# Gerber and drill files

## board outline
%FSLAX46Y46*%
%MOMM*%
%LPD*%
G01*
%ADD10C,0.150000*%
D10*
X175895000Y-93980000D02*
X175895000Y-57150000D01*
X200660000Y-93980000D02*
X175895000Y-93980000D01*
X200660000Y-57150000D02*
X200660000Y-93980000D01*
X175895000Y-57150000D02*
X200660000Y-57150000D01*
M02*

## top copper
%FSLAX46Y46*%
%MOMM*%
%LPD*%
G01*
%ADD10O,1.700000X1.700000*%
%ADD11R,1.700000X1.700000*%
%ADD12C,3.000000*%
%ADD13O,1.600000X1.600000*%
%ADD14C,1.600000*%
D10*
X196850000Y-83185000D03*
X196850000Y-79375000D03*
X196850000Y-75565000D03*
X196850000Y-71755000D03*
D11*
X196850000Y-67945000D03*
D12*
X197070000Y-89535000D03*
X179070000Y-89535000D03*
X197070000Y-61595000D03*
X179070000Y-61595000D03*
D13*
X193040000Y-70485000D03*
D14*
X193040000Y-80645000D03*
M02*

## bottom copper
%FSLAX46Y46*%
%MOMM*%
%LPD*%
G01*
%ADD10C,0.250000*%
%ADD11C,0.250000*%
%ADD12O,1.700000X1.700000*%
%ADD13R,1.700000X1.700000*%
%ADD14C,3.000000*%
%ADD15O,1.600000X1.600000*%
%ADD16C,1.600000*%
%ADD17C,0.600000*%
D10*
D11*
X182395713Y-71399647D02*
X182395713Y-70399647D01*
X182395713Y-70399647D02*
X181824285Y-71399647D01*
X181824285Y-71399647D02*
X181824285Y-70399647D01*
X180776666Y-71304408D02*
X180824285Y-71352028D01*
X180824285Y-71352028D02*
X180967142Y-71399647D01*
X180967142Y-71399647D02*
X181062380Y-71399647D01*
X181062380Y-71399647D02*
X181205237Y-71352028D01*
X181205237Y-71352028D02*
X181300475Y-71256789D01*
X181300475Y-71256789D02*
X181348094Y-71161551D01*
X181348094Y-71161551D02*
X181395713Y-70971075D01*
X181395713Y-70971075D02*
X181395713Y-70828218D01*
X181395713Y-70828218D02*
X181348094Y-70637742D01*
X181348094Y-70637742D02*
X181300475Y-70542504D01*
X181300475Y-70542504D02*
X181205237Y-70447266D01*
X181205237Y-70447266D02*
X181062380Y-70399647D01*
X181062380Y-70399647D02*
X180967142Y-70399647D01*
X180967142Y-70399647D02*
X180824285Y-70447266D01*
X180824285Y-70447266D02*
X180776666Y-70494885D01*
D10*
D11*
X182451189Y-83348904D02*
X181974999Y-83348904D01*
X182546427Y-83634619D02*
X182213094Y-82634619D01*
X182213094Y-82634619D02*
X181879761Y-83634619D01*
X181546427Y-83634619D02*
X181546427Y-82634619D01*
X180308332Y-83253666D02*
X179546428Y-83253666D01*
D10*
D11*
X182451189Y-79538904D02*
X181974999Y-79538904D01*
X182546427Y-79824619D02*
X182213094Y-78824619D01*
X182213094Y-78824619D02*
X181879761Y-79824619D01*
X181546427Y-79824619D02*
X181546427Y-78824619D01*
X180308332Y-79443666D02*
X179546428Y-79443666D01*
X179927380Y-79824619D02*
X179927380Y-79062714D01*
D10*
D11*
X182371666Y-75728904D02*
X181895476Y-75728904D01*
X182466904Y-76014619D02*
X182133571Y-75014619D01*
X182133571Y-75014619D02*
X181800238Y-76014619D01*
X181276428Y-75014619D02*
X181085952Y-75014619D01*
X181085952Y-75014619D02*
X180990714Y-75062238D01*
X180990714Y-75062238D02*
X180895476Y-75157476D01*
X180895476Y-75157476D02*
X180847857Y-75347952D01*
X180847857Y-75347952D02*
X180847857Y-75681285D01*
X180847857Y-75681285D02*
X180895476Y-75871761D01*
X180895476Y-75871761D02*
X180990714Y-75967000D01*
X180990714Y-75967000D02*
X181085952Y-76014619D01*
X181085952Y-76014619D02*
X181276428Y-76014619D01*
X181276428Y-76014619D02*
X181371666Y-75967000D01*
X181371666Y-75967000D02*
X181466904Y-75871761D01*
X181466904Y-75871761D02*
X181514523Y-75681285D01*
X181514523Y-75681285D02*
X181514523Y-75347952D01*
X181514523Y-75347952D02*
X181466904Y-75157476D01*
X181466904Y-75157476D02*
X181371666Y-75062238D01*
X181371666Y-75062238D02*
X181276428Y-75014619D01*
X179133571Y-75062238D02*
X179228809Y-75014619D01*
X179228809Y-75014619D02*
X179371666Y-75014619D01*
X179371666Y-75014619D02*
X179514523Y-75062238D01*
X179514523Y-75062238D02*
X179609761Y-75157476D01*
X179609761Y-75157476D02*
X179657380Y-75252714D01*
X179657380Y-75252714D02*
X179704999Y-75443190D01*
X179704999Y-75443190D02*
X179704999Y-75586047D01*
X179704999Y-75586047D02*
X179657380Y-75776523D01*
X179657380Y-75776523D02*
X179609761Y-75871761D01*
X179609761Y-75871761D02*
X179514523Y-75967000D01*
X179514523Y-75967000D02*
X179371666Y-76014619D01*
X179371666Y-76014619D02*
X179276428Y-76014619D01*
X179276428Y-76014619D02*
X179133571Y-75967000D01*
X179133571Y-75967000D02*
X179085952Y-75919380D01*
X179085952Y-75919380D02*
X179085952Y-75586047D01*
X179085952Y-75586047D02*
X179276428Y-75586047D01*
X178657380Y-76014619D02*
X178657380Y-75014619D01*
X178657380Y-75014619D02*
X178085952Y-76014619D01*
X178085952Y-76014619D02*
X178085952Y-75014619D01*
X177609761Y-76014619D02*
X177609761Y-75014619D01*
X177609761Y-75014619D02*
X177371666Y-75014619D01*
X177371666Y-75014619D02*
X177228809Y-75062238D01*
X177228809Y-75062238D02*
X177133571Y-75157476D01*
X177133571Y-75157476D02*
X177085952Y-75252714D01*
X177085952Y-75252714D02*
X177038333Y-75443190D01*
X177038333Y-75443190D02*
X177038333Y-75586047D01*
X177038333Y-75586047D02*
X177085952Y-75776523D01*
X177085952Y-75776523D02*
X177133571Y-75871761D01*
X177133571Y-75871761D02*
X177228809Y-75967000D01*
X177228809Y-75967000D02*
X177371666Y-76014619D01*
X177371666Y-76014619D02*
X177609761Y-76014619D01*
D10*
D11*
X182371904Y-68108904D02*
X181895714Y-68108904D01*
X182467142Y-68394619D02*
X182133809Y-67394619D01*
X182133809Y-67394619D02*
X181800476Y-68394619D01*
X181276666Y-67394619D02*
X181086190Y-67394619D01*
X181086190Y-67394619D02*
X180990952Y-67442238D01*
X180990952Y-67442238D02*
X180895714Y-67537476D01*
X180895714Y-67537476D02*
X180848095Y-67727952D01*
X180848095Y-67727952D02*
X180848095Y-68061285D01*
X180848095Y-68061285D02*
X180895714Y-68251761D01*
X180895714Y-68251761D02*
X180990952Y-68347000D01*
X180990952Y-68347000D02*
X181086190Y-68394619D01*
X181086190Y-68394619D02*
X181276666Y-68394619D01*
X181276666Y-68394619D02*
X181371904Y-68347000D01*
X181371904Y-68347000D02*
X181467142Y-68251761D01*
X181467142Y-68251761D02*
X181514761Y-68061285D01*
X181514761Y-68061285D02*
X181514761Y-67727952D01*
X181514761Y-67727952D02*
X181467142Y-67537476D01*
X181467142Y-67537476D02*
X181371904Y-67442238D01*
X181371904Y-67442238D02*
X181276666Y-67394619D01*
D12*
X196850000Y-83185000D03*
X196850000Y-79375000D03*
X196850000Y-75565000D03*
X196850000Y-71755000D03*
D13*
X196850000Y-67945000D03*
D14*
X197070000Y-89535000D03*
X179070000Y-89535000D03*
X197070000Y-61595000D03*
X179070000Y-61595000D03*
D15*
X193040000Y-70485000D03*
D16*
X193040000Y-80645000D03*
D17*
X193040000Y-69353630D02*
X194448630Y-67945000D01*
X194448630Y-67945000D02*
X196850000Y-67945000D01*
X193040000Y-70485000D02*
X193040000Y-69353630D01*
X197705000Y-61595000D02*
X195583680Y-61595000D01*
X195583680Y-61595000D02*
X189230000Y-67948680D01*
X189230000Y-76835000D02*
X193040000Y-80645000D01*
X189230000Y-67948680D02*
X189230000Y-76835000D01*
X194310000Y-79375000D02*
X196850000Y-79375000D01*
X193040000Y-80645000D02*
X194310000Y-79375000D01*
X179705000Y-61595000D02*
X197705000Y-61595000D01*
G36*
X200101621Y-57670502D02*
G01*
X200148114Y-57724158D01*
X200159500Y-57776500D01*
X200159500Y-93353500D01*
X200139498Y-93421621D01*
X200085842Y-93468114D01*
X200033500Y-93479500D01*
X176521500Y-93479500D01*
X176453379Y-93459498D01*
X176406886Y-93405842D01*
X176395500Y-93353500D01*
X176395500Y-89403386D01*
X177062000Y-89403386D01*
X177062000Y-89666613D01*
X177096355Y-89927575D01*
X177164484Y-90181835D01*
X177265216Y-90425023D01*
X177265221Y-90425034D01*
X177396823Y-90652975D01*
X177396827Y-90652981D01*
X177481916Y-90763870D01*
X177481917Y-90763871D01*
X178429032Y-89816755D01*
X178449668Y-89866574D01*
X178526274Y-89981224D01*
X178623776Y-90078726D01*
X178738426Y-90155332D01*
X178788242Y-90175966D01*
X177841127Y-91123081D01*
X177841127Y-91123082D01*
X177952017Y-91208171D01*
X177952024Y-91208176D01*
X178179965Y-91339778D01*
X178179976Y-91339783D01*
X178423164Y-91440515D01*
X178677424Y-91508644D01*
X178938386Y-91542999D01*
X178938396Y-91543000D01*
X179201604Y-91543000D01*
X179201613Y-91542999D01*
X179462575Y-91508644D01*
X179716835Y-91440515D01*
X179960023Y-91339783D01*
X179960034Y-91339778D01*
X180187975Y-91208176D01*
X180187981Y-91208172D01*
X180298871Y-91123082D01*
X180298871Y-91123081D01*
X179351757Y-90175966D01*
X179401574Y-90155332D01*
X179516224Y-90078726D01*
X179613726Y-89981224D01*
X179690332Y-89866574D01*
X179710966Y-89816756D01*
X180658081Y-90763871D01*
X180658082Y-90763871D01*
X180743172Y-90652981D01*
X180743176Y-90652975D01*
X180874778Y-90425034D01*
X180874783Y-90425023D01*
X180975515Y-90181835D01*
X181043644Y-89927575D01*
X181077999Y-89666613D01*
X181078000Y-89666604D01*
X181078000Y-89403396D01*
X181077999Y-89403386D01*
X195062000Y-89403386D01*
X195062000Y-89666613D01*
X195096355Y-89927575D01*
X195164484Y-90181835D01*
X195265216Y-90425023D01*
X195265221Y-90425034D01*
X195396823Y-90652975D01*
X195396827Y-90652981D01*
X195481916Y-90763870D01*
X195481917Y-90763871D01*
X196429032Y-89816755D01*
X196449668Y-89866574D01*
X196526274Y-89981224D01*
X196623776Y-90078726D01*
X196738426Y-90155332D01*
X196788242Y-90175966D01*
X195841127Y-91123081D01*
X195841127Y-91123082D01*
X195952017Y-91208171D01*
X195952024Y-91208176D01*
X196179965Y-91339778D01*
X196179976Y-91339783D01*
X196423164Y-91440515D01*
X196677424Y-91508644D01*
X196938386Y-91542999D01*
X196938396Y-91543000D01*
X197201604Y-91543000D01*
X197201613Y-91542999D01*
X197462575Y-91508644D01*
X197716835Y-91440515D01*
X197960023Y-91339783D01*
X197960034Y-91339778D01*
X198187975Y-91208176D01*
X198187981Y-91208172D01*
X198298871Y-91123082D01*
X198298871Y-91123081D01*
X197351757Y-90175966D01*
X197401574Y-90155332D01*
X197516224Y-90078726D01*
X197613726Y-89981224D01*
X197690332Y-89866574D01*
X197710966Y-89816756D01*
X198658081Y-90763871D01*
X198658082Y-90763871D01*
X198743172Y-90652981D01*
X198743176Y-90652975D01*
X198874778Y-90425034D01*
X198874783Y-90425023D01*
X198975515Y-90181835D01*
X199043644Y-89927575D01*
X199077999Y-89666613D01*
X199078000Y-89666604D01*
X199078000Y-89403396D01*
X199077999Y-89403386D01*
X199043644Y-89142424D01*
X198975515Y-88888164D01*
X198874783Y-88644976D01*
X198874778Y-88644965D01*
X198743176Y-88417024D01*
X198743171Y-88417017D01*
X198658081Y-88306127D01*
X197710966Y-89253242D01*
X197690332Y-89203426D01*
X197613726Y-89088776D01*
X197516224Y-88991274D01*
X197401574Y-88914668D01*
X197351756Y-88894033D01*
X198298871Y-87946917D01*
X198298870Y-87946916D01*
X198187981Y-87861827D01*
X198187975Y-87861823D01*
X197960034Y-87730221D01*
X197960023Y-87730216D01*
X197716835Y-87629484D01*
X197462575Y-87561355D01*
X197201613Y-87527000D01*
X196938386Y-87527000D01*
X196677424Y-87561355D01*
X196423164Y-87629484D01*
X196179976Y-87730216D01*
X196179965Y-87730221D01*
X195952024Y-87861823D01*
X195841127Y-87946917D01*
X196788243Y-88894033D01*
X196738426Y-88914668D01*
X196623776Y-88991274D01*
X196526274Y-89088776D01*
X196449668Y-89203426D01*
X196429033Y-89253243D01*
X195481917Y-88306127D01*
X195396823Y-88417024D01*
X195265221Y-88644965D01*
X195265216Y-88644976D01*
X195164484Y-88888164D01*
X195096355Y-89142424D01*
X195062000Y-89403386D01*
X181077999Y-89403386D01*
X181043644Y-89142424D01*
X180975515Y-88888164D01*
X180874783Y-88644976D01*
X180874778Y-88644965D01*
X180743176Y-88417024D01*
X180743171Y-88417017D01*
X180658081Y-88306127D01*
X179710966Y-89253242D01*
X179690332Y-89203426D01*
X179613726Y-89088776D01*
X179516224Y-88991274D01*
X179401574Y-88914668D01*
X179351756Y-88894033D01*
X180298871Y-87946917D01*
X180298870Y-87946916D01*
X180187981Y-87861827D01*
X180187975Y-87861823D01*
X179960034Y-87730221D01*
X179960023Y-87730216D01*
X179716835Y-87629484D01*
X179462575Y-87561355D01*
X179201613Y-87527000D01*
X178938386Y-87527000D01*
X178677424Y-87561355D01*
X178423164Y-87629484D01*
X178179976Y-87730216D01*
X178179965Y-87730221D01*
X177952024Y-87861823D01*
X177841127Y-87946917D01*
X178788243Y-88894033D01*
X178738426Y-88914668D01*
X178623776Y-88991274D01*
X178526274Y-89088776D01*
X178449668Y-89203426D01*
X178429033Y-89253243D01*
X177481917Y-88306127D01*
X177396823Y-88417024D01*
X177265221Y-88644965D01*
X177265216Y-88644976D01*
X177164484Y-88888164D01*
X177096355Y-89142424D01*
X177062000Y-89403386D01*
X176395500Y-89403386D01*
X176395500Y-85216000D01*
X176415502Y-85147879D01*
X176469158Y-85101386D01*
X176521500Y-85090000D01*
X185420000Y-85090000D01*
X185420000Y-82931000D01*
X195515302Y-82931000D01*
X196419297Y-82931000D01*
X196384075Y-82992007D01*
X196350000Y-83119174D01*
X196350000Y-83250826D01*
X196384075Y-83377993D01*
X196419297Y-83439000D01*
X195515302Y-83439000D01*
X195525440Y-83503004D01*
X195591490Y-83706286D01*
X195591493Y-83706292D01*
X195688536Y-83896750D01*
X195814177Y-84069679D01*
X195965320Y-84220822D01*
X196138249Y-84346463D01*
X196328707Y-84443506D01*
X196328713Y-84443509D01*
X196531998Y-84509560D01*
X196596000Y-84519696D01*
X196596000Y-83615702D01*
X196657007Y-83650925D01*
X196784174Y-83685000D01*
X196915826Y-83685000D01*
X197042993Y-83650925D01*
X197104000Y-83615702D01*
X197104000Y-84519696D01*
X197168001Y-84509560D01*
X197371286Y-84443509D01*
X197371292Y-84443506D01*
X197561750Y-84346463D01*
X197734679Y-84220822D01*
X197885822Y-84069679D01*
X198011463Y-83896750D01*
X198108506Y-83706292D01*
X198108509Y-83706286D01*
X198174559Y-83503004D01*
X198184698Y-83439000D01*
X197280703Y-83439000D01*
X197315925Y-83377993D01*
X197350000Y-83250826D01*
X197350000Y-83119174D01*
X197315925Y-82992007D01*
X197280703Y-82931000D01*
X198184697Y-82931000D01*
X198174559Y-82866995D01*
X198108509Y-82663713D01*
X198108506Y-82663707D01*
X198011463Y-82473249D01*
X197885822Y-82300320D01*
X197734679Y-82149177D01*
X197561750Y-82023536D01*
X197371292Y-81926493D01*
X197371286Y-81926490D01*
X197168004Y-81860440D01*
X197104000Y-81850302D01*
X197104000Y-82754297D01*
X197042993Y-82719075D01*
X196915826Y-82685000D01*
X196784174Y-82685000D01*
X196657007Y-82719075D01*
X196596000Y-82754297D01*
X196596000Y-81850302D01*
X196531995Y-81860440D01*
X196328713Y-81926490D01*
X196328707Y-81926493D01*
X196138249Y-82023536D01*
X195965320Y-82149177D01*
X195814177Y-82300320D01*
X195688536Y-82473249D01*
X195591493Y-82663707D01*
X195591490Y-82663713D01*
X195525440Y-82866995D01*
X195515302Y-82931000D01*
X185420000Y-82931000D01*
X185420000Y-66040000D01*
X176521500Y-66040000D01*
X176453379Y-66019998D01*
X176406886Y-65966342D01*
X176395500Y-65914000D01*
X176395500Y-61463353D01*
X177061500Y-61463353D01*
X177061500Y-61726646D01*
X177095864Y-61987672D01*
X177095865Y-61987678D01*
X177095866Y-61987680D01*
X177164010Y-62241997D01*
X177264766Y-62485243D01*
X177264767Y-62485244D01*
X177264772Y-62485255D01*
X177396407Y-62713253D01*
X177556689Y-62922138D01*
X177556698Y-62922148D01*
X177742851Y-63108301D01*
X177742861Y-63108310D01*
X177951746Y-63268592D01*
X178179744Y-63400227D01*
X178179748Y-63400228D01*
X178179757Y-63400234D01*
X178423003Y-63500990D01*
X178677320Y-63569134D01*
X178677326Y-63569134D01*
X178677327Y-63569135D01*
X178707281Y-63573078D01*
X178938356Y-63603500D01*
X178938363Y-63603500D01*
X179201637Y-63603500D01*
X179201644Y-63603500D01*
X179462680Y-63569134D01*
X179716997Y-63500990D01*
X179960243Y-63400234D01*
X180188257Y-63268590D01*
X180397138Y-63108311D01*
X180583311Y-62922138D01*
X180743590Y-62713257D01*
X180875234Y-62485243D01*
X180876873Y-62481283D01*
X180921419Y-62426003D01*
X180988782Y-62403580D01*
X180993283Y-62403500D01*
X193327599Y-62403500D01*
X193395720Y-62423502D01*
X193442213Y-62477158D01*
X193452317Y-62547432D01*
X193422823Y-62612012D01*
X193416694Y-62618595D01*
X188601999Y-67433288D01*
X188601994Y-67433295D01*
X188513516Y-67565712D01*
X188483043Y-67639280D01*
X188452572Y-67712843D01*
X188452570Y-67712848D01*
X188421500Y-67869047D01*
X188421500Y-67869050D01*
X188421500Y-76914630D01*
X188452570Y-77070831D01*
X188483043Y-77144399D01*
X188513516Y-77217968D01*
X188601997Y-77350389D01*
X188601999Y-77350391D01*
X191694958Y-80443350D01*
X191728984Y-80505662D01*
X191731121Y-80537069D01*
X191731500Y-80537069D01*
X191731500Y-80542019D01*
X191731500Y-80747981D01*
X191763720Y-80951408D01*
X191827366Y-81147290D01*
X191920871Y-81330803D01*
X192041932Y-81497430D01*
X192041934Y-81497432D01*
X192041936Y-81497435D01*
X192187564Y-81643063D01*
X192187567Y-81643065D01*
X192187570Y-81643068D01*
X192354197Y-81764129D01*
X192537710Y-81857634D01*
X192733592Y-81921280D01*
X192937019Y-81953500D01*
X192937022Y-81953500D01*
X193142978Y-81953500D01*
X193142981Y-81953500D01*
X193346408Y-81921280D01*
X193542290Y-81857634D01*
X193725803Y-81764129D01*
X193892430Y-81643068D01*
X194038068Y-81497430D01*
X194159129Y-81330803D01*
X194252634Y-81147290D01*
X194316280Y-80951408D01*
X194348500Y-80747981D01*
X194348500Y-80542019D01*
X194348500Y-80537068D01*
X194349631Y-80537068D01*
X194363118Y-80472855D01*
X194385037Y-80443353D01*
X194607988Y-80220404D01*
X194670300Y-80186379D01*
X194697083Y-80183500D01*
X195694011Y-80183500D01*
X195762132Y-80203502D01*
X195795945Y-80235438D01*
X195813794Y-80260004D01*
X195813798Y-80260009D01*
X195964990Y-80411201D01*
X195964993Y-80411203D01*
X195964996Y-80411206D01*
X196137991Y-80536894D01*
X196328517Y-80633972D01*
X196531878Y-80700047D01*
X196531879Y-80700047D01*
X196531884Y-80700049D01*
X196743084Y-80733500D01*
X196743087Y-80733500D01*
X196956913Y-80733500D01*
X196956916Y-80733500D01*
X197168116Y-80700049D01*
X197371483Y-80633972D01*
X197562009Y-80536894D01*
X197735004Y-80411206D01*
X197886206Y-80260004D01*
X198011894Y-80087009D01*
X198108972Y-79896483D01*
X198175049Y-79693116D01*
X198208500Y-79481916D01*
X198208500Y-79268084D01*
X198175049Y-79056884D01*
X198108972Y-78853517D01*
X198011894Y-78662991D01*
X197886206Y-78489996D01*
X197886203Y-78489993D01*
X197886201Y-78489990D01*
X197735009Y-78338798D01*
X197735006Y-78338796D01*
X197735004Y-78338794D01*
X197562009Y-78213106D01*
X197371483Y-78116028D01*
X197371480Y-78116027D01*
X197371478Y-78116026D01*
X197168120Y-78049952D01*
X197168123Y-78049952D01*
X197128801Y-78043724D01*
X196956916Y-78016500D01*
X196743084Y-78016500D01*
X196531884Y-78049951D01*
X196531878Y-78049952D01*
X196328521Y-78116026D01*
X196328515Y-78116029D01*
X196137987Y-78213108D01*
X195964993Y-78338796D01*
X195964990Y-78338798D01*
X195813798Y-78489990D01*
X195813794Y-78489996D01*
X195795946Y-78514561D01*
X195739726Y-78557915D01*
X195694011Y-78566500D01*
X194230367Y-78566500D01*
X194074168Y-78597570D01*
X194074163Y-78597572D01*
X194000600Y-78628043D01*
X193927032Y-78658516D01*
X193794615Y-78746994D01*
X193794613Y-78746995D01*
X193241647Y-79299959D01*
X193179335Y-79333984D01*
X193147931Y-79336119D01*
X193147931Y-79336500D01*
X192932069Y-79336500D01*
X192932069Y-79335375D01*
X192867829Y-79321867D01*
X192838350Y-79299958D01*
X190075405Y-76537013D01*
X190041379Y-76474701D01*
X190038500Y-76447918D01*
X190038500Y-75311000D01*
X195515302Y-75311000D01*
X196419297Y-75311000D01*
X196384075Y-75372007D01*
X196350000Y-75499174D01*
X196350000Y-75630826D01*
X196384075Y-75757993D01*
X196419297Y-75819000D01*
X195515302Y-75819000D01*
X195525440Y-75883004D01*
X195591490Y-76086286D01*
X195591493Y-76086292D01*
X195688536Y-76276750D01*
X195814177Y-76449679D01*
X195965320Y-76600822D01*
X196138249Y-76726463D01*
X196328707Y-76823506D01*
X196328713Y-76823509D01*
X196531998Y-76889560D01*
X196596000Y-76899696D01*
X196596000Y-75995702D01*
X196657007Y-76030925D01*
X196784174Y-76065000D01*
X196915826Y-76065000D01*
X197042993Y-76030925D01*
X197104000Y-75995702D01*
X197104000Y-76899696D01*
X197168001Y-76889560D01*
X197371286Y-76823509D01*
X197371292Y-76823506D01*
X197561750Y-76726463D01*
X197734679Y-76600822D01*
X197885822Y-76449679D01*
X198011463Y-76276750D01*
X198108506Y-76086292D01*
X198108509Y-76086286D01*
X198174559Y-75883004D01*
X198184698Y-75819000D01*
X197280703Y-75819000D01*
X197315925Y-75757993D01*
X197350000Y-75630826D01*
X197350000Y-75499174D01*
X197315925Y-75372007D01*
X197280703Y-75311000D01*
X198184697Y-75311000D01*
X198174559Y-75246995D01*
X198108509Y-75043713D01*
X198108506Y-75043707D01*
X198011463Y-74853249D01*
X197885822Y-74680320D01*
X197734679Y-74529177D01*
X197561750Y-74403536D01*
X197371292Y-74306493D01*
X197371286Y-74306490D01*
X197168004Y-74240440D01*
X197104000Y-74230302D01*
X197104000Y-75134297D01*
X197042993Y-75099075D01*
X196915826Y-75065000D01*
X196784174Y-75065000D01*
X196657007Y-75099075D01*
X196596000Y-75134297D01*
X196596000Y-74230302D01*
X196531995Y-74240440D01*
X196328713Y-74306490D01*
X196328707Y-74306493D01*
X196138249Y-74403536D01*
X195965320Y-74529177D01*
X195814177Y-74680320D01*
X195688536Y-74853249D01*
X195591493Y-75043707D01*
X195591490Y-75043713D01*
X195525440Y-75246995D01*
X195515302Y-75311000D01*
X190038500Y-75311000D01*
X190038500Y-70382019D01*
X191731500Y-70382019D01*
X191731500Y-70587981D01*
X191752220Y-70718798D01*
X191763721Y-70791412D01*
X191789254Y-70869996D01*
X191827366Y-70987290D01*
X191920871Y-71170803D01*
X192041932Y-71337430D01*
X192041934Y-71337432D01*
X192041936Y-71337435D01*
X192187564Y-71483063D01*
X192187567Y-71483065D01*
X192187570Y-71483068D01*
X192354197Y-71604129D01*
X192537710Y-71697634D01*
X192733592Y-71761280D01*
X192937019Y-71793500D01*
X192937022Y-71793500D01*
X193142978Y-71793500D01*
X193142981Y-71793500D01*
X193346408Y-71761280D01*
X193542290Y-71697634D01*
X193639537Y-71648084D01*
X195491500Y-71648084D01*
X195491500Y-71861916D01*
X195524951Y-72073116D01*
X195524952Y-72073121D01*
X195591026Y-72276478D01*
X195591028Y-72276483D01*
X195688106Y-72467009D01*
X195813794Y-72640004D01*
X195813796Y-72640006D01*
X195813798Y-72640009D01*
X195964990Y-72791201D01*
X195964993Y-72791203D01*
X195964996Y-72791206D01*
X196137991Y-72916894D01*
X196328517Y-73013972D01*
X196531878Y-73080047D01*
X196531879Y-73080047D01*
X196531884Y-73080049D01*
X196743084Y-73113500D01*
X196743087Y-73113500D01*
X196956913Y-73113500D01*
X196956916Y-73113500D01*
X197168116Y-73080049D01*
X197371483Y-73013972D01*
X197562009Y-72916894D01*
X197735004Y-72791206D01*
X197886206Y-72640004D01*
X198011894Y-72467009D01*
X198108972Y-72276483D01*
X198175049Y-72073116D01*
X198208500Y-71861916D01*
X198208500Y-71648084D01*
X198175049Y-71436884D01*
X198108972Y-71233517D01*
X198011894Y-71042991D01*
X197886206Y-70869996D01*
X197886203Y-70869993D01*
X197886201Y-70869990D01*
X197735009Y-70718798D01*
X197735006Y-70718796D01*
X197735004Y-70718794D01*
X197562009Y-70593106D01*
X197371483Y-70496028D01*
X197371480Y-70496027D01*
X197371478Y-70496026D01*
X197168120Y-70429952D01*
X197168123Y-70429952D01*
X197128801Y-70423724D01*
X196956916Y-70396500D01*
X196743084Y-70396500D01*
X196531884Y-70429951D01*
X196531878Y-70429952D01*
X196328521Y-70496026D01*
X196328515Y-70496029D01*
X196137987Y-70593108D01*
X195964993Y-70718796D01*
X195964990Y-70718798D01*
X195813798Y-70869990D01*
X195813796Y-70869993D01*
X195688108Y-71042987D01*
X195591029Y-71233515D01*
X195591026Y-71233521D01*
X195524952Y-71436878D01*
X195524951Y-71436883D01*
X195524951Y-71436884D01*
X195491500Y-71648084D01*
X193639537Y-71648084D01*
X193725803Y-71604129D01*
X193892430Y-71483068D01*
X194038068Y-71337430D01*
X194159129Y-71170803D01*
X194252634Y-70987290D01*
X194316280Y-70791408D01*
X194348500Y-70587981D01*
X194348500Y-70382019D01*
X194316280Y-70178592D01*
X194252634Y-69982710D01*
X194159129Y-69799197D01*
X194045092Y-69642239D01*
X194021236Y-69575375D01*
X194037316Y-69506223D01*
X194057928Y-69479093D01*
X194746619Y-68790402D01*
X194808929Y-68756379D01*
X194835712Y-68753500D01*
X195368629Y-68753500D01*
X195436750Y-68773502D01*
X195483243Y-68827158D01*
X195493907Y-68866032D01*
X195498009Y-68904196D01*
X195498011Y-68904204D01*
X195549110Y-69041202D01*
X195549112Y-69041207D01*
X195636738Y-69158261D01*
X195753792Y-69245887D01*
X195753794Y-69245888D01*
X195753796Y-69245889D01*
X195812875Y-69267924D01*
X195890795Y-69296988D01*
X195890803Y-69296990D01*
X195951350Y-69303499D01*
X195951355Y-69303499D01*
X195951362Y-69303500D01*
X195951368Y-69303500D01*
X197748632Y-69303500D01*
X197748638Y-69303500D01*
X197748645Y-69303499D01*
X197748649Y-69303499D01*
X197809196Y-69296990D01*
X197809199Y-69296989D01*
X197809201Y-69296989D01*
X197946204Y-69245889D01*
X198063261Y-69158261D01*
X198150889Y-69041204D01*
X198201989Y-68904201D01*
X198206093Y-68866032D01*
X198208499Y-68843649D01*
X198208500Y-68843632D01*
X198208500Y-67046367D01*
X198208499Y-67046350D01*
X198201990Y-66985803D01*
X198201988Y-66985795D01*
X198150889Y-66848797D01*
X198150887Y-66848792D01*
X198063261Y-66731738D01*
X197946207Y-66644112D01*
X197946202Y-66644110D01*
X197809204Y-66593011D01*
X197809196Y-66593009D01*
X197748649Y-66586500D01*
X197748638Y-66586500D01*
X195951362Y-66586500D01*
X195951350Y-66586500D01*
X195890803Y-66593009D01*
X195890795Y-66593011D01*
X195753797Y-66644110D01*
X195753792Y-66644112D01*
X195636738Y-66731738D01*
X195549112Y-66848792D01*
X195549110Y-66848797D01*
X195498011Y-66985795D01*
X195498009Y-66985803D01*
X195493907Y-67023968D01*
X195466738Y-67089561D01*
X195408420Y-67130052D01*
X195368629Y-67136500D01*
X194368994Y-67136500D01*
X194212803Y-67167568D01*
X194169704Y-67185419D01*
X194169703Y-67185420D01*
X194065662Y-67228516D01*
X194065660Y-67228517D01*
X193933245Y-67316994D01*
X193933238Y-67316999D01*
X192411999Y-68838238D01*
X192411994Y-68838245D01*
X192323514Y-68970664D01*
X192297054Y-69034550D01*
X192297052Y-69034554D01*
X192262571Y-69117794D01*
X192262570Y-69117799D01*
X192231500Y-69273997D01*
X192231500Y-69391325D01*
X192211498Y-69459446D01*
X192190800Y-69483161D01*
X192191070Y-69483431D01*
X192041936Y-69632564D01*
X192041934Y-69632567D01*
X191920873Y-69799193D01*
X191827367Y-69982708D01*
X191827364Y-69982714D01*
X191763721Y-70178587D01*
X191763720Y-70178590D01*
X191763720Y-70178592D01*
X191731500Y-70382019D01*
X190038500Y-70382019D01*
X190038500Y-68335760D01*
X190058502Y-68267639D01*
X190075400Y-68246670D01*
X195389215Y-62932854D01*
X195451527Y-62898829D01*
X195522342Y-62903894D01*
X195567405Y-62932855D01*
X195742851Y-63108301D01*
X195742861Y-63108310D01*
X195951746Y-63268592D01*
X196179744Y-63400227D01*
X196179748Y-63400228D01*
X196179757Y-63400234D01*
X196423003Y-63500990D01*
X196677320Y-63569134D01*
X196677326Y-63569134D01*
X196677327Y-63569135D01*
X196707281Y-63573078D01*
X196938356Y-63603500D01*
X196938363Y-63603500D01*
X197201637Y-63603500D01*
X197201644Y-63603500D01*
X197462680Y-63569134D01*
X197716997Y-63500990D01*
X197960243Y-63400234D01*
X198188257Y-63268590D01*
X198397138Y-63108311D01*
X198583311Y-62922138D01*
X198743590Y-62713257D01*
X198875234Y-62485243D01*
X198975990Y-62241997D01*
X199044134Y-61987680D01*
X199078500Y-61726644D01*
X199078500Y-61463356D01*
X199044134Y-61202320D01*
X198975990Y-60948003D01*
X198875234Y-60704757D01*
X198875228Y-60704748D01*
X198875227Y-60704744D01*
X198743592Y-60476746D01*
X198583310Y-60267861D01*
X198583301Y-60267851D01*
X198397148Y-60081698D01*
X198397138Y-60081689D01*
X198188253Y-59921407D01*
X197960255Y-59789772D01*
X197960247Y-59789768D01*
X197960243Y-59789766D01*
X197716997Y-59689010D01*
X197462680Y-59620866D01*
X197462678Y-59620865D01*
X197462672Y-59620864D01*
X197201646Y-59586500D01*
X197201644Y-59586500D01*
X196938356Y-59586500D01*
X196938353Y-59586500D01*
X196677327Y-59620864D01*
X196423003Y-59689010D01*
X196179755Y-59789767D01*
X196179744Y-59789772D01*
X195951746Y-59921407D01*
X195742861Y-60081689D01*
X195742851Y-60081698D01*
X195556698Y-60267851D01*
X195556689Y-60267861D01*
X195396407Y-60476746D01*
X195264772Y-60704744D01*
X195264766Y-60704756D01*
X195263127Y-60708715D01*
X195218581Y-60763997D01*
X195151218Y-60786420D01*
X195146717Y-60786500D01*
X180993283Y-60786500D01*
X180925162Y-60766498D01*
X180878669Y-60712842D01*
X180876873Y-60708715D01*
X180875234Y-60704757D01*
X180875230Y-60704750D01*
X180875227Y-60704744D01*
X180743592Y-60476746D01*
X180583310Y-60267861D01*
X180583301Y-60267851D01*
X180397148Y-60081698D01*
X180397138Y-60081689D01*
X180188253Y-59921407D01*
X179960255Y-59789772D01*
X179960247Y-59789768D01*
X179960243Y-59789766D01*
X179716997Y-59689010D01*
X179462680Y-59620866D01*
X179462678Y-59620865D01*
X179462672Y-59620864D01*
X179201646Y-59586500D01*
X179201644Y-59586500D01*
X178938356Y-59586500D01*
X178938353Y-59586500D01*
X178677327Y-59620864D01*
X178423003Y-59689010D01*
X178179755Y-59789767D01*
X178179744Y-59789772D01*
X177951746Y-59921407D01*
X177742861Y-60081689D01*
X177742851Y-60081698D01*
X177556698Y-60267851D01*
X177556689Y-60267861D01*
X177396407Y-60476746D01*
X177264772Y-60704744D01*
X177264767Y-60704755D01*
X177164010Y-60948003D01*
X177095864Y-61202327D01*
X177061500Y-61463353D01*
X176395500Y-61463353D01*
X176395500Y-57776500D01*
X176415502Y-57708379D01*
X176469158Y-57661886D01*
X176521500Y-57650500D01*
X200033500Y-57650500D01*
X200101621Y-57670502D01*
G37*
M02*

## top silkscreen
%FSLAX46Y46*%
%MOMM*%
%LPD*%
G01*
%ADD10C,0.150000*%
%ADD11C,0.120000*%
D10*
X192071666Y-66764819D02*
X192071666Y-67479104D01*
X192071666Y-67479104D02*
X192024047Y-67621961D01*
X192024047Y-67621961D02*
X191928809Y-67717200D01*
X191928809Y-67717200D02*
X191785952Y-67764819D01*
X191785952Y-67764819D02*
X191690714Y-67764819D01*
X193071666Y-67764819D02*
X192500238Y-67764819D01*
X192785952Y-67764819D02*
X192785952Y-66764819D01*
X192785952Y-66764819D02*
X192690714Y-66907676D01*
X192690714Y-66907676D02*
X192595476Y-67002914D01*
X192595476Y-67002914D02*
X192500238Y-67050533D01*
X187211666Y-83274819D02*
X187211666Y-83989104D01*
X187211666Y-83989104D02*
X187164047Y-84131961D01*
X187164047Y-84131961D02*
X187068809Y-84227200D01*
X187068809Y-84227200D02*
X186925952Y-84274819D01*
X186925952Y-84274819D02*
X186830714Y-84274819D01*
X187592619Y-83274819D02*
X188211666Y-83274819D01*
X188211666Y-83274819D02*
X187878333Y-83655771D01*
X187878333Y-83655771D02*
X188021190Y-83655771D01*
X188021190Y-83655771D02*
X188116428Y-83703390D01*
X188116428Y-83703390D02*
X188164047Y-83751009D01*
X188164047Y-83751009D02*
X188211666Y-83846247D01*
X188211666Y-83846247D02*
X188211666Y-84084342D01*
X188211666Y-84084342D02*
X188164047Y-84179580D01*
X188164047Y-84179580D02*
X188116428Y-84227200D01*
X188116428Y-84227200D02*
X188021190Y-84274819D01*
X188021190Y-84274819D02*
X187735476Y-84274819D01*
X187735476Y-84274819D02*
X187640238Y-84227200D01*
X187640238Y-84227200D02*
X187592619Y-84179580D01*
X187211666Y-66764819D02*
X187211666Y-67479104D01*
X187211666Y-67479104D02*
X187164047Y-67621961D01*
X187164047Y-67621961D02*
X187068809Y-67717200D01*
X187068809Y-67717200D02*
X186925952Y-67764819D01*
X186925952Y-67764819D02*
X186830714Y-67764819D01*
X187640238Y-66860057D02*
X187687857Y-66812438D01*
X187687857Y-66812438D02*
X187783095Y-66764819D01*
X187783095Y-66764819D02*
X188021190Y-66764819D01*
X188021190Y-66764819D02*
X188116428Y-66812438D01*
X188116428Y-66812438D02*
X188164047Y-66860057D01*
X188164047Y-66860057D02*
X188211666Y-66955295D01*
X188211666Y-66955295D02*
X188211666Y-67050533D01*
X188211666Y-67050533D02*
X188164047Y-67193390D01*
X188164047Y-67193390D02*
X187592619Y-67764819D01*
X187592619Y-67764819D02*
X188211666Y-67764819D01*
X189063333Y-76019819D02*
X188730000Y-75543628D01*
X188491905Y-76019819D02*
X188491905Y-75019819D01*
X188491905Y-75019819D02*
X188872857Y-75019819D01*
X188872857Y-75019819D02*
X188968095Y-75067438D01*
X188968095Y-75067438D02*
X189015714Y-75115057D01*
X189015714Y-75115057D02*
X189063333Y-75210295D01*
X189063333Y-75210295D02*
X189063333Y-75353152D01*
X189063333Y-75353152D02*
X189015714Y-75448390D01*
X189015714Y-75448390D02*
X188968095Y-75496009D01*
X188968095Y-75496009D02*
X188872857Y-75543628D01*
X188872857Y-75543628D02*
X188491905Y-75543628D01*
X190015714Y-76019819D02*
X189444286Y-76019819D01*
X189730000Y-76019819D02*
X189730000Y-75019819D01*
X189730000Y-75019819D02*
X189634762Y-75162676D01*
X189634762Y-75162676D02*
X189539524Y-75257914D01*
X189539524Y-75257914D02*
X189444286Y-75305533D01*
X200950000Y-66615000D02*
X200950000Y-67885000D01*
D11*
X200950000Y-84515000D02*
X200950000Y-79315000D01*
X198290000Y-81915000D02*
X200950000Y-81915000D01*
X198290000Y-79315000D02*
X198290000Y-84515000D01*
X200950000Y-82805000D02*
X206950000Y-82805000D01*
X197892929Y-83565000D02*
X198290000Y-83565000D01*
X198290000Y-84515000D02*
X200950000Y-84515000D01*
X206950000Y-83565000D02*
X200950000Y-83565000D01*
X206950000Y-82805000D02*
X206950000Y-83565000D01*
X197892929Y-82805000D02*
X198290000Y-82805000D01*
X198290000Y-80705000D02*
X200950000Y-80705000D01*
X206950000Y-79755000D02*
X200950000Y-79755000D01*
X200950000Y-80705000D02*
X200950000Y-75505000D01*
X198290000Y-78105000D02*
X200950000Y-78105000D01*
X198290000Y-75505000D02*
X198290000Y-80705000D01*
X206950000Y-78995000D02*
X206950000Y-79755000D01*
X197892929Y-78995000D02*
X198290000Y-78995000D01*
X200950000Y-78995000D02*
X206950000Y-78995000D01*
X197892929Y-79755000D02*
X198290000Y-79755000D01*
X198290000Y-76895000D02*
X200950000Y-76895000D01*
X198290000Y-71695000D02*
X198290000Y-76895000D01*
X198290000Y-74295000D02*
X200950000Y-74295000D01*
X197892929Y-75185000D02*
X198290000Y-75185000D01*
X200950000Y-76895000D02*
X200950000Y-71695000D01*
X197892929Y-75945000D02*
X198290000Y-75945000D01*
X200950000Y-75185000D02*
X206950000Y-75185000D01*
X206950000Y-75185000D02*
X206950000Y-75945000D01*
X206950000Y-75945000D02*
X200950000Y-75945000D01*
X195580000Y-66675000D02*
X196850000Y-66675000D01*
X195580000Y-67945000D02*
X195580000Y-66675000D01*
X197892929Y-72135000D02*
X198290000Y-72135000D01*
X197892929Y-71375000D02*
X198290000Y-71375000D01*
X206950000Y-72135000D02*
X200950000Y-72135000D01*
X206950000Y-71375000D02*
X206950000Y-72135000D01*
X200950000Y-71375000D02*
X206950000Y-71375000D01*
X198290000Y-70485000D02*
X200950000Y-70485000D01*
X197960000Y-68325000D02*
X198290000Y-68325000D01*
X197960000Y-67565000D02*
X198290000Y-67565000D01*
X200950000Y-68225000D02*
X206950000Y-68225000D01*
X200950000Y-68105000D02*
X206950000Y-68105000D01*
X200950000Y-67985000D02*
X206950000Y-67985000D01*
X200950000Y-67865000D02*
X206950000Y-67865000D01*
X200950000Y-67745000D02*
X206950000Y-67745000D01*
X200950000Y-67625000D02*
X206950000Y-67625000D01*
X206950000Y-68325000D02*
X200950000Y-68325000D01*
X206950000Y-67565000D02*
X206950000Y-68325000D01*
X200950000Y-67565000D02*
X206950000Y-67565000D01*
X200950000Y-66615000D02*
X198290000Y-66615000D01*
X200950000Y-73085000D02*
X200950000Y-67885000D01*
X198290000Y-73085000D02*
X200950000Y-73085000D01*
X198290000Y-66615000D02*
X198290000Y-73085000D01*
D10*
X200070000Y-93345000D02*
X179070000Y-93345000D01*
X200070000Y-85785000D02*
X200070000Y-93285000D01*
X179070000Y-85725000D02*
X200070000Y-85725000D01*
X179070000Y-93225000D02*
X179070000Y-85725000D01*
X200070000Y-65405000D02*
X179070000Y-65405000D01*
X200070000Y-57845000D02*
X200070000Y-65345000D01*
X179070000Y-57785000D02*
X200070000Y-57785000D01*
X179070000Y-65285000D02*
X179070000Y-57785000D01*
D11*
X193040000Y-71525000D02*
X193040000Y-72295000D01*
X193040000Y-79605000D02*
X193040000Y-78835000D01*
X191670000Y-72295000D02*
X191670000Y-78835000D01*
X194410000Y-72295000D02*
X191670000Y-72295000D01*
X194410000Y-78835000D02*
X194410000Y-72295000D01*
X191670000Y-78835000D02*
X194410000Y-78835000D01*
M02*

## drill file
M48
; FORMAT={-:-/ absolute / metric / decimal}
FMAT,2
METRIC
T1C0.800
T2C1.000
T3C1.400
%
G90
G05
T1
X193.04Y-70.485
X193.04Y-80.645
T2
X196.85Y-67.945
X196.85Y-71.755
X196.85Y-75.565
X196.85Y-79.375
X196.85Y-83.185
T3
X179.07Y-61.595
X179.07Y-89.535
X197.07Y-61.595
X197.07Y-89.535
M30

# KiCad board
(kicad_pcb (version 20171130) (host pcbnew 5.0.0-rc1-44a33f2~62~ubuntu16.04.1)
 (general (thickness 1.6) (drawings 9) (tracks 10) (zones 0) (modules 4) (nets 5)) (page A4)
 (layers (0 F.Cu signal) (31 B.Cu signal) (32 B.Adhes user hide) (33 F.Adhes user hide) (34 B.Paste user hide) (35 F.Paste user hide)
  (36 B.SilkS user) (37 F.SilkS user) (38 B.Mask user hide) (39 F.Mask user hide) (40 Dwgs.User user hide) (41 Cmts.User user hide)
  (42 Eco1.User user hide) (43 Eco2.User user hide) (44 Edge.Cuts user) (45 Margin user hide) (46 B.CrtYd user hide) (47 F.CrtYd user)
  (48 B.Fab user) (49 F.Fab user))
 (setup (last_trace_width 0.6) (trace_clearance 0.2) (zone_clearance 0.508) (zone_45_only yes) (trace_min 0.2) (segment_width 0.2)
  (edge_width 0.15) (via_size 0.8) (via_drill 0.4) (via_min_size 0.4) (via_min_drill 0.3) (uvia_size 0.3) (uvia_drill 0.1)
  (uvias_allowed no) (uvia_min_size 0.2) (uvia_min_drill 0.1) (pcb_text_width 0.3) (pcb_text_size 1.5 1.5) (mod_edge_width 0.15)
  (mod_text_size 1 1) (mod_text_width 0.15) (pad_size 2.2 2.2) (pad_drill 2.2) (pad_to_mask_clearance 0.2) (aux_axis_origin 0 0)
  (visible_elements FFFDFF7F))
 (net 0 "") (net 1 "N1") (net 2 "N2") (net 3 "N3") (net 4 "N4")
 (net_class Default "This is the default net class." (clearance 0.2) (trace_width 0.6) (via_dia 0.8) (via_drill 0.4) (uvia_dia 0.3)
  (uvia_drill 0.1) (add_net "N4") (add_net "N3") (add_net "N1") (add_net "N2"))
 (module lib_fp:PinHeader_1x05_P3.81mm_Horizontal (layer F.Cu) (at 196.85 67.945)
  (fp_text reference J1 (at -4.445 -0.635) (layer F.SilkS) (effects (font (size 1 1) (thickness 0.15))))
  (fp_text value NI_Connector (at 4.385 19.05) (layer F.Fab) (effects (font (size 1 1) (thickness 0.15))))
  (fp_line (start 4.1 -1.33) (end 4.1 -0.06) (layer F.SilkS) (width 0.15))
  (fp_line (start 4.1 16.57) (end 4.1 11.37) (layer F.SilkS) (width 0.12))
  (fp_line (start 1.44 13.97) (end 4.1 13.97) (layer F.SilkS) (width 0.12))
  (fp_line (start 1.44 11.37) (end 1.44 16.57) (layer F.SilkS) (width 0.12))
  (fp_line (start 4.1 14.86) (end 10.1 14.86) (layer F.SilkS) (width 0.12))
  (fp_line (start 1.042929 15.62) (end 1.44 15.62) (layer F.SilkS) (width 0.12))
  (fp_line (start 1.44 16.57) (end 4.1 16.57) (layer F.SilkS) (width 0.12))
  (fp_line (start 10.1 15.62) (end 4.1 15.62) (layer F.SilkS) (width 0.12))
  (fp_line (start 10.1 14.86) (end 10.1 15.62) (layer F.SilkS) (width 0.12))
  (fp_line (start 1.042929 14.86) (end 1.44 14.86) (layer F.SilkS) (width 0.12))
  (fp_line (start 1.44 12.76) (end 4.1 12.76) (layer F.SilkS) (width 0.12))
  (fp_line (start 10.1 11.81) (end 4.1 11.81) (layer F.SilkS) (width 0.12))
  (fp_line (start 4.1 12.76) (end 4.1 7.56) (layer F.SilkS) (width 0.12))
  (fp_line (start 1.44 10.16) (end 4.1 10.16) (layer F.SilkS) (width 0.12))
  (fp_line (start 1.44 7.56) (end 1.44 12.76) (layer F.SilkS) (width 0.12))
  (fp_line (start 10.1 11.05) (end 10.1 11.81) (layer F.SilkS) (width 0.12))
  (fp_line (start 1.042929 11.05) (end 1.44 11.05) (layer F.SilkS) (width 0.12))
  (fp_line (start 4.1 11.05) (end 10.1 11.05) (layer F.SilkS) (width 0.12))
  (fp_line (start 1.042929 11.81) (end 1.44 11.81) (layer F.SilkS) (width 0.12))
  (fp_line (start 1.44 8.95) (end 4.1 8.95) (layer F.SilkS) (width 0.12))
  (fp_line (start 1.44 3.75) (end 1.44 8.95) (layer F.SilkS) (width 0.12))
  (fp_line (start 1.44 6.35) (end 4.1 6.35) (layer F.SilkS) (width 0.12))
  (fp_line (start 1.042929 7.24) (end 1.44 7.24) (layer F.SilkS) (width 0.12))
  (fp_line (start 4.1 8.95) (end 4.1 3.75) (layer F.SilkS) (width 0.12))
  (fp_line (start 1.042929 8) (end 1.44 8) (layer F.SilkS) (width 0.12))
  (fp_line (start 4.1 7.24) (end 10.1 7.24) (layer F.SilkS) (width 0.12))
  (fp_line (start 10.1 7.24) (end 10.1 8) (layer F.SilkS) (width 0.12))
  (fp_line (start 10.1 8) (end 4.1 8) (layer F.SilkS) (width 0.12))
  (fp_line (start -1.27 -1.27) (end 0 -1.27) (layer F.SilkS) (width 0.12))
  (fp_line (start -1.27 0) (end -1.27 -1.27) (layer F.SilkS) (width 0.12))
  (fp_line (start 1.042929 4.19) (end 1.44 4.19) (layer F.SilkS) (width 0.12))
  (fp_line (start 1.042929 3.43) (end 1.44 3.43) (layer F.SilkS) (width 0.12))
  (fp_line (start 10.1 4.19) (end 4.1 4.19) (layer F.SilkS) (width 0.12))
  (fp_line (start 10.1 3.43) (end 10.1 4.19) (layer F.SilkS) (width 0.12))
  (fp_line (start 4.1 3.43) (end 10.1 3.43) (layer F.SilkS) (width 0.12))
  (fp_line (start 1.44 2.54) (end 4.1 2.54) (layer F.SilkS) (width 0.12))
  (fp_line (start 1.11 0.38) (end 1.44 0.38) (layer F.SilkS) (width 0.12))
  (fp_line (start 1.11 -0.38) (end 1.44 -0.38) (layer F.SilkS) (width 0.12))
  (fp_line (start 4.1 0.28) (end 10.1 0.28) (layer F.SilkS) (width 0.12))
  (fp_line (start 4.1 0.16) (end 10.1 0.16) (layer F.SilkS) (width 0.12))
  (fp_line (start 4.1 0.04) (end 10.1 0.04) (layer F.SilkS) (width 0.12))
  (fp_line (start 4.1 -0.08) (end 10.1 -0.08) (layer F.SilkS) (width 0.12))
  (fp_line (start 4.1 -0.2) (end 10.1 -0.2) (layer F.SilkS) (width 0.12))
  (fp_line (start 4.1 -0.32) (end 10.1 -0.32) (layer F.SilkS) (width 0.12))
  (fp_line (start 10.1 0.38) (end 4.1 0.38) (layer F.SilkS) (width 0.12))
  (fp_line (start 10.1 -0.38) (end 10.1 0.38) (layer F.SilkS) (width 0.12))
  (fp_line (start 4.1 -0.38) (end 10.1 -0.38) (layer F.SilkS) (width 0.12))
  (fp_line (start 4.1 -1.33) (end 1.44 -1.33) (layer F.SilkS) (width 0.12))
  (fp_line (start 4.1 5.14) (end 4.1 -0.06) (layer F.SilkS) (width 0.12))
  (fp_line (start 1.44 5.14) (end 4.1 5.14) (layer F.SilkS) (width 0.12))
  (fp_line (start 1.44 -1.33) (end 1.44 5.14) (layer F.SilkS) (width 0.12))
  (pad 5 thru_hole oval (at 0 15.24) (size 1.7 1.7) (drill 1) (layers *.Cu *.Mask) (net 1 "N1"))
  (pad 4 thru_hole oval (at 0 11.43) (size 1.7 1.7) (drill 1) (layers *.Cu *.Mask) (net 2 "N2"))
  (pad 3 thru_hole oval (at 0 7.62) (size 1.7 1.7) (drill 1) (layers *.Cu *.Mask) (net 1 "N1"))
  (pad 2 thru_hole oval (at 0 3.81) (size 1.7 1.7) (drill 1) (layers *.Cu *.Mask) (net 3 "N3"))
  (pad 1 thru_hole rect (at 0 0) (size 1.7 1.7) (drill 1) (layers *.Cu *.Mask) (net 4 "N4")))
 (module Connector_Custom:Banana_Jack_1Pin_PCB (layer F.Cu) (at 179.07 89.535 90)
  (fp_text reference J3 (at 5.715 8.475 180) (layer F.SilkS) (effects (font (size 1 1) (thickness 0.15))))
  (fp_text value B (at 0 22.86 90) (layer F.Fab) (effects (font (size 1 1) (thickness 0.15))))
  (fp_line (start -3.81 21) (end -3.81 0) (layer F.SilkS) (width 0.15))
  (fp_line (start 3.75 21) (end -3.75 21) (layer F.SilkS) (width 0.15))
  (fp_line (start 3.81 0) (end 3.81 21) (layer F.SilkS) (width 0.15))
  (fp_line (start -3.69 0) (end 3.81 0) (layer F.SilkS) (width 0.15))
  (pad 1 thru_hole circle (at 0 18 90) (size 3 3) (drill 1.4) (layers *.Cu *.Mask) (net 1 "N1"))
  (pad 1 thru_hole circle (at 0 0 90) (size 3 3) (drill 1.4) (layers *.Cu *.Mask) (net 1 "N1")))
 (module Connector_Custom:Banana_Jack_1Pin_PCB (layer F.Cu) (at 179.07 61.595 90)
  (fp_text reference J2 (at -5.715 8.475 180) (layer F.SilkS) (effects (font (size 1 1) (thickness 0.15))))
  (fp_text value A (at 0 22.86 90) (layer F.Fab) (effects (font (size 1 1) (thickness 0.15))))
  (fp_line (start -3.81 21) (end -3.81 0) (layer F.SilkS) (width 0.15))
  (fp_line (start 3.75 21) (end -3.75 21) (layer F.SilkS) (width 0.15))
  (fp_line (start 3.81 0) (end 3.81 21) (layer F.SilkS) (width 0.15))
  (fp_line (start -3.69 0) (end 3.81 0) (layer F.SilkS) (width 0.15))
  (pad 1 thru_hole circle (at 0 18 90) (size 3 3) (drill 1.4) (layers *.Cu *.Mask) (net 2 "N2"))
  (pad 1 thru_hole circle (at 0 0 90) (size 3 3) (drill 1.4) (layers *.Cu *.Mask) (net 2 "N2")))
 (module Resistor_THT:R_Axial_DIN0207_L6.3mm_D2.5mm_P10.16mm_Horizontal (layer F.Cu) (at 193.04 80.645 90)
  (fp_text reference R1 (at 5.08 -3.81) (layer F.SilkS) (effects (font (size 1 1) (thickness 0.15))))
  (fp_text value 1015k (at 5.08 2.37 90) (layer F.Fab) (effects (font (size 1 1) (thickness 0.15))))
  (fp_line (start 9.12 0) (end 8.35 0) (layer F.SilkS) (width 0.12))
  (fp_line (start 1.04 0) (end 1.81 0) (layer F.SilkS) (width 0.12))
  (fp_line (start 8.35 -1.37) (end 1.81 -1.37) (layer F.SilkS) (width 0.12))
  (fp_line (start 8.35 1.37) (end 8.35 -1.37) (layer F.SilkS) (width 0.12))
  (fp_line (start 1.81 1.37) (end 8.35 1.37) (layer F.SilkS) (width 0.12))
  (fp_line (start 1.81 -1.37) (end 1.81 1.37) (layer F.SilkS) (width 0.12))
  (pad 2 thru_hole oval (at 10.16 0 90) (size 1.6 1.6) (drill 0.8) (layers *.Cu *.Mask) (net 4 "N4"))
  (pad 1 thru_hole circle (at 0 0 90) (size 1.6 1.6) (drill 0.8) (layers *.Cu *.Mask) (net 2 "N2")))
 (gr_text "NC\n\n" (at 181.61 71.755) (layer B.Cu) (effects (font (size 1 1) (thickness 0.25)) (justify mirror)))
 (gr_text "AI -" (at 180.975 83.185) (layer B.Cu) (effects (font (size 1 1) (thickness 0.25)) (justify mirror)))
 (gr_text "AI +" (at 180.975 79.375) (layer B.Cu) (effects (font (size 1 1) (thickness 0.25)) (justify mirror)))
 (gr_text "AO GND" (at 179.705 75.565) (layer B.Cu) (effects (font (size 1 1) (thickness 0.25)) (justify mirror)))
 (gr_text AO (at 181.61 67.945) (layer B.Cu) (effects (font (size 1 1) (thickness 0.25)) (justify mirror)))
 (gr_line (start 175.895 93.98) (end 175.895 57.15) (layer Edge.Cuts) (width 0.15))
 (gr_line (start 200.66 93.98) (end 175.895 93.98) (layer Edge.Cuts) (width 0.15))
 (gr_line (start 200.66 57.15) (end 200.66 93.98) (layer Edge.Cuts) (width 0.15))
 (gr_line (start 175.895 57.15) (end 200.66 57.15) (layer Edge.Cuts) (width 0.15))
 (segment (start 193.04 69.35363) (end 194.44863 67.945) (width 0.6) (layer B.Cu) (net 4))
 (segment (start 194.44863 67.945) (end 196.85 67.945) (width 0.6) (layer B.Cu) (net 4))
 (segment (start 193.04 70.485) (end 193.04 69.35363) (width 0.6) (layer B.Cu) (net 4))
 (segment (start 197.705 61.595) (end 195.58368 61.595) (width 0.6) (layer B.Cu) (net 2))
 (segment (start 195.58368 61.595) (end 189.23 67.94868) (width 0.6) (layer B.Cu) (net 2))
 (segment (start 189.23 76.835) (end 193.04 80.645) (width 0.6) (layer B.Cu) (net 2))
 (segment (start 189.23 67.94868) (end 189.23 76.835) (width 0.6) (layer B.Cu) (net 2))
 (segment (start 194.31 79.375) (end 196.85 79.375) (width 0.6) (layer B.Cu) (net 2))
 (segment (start 193.04 80.645) (end 194.31 79.375) (width 0.6) (layer B.Cu) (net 2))
 (segment (start 179.705 61.595) (end 197.705 61.595) (width 0.6) (layer B.Cu) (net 2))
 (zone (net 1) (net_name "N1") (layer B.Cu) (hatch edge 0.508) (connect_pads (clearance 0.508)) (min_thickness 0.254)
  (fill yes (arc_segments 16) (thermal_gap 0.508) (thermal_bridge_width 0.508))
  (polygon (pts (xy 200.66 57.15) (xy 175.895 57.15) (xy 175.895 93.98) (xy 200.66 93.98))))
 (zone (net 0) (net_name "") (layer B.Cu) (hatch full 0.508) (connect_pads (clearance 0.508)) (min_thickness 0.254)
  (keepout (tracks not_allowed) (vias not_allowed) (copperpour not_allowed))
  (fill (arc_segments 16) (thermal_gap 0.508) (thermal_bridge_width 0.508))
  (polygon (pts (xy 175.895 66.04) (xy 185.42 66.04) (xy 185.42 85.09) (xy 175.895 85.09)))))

